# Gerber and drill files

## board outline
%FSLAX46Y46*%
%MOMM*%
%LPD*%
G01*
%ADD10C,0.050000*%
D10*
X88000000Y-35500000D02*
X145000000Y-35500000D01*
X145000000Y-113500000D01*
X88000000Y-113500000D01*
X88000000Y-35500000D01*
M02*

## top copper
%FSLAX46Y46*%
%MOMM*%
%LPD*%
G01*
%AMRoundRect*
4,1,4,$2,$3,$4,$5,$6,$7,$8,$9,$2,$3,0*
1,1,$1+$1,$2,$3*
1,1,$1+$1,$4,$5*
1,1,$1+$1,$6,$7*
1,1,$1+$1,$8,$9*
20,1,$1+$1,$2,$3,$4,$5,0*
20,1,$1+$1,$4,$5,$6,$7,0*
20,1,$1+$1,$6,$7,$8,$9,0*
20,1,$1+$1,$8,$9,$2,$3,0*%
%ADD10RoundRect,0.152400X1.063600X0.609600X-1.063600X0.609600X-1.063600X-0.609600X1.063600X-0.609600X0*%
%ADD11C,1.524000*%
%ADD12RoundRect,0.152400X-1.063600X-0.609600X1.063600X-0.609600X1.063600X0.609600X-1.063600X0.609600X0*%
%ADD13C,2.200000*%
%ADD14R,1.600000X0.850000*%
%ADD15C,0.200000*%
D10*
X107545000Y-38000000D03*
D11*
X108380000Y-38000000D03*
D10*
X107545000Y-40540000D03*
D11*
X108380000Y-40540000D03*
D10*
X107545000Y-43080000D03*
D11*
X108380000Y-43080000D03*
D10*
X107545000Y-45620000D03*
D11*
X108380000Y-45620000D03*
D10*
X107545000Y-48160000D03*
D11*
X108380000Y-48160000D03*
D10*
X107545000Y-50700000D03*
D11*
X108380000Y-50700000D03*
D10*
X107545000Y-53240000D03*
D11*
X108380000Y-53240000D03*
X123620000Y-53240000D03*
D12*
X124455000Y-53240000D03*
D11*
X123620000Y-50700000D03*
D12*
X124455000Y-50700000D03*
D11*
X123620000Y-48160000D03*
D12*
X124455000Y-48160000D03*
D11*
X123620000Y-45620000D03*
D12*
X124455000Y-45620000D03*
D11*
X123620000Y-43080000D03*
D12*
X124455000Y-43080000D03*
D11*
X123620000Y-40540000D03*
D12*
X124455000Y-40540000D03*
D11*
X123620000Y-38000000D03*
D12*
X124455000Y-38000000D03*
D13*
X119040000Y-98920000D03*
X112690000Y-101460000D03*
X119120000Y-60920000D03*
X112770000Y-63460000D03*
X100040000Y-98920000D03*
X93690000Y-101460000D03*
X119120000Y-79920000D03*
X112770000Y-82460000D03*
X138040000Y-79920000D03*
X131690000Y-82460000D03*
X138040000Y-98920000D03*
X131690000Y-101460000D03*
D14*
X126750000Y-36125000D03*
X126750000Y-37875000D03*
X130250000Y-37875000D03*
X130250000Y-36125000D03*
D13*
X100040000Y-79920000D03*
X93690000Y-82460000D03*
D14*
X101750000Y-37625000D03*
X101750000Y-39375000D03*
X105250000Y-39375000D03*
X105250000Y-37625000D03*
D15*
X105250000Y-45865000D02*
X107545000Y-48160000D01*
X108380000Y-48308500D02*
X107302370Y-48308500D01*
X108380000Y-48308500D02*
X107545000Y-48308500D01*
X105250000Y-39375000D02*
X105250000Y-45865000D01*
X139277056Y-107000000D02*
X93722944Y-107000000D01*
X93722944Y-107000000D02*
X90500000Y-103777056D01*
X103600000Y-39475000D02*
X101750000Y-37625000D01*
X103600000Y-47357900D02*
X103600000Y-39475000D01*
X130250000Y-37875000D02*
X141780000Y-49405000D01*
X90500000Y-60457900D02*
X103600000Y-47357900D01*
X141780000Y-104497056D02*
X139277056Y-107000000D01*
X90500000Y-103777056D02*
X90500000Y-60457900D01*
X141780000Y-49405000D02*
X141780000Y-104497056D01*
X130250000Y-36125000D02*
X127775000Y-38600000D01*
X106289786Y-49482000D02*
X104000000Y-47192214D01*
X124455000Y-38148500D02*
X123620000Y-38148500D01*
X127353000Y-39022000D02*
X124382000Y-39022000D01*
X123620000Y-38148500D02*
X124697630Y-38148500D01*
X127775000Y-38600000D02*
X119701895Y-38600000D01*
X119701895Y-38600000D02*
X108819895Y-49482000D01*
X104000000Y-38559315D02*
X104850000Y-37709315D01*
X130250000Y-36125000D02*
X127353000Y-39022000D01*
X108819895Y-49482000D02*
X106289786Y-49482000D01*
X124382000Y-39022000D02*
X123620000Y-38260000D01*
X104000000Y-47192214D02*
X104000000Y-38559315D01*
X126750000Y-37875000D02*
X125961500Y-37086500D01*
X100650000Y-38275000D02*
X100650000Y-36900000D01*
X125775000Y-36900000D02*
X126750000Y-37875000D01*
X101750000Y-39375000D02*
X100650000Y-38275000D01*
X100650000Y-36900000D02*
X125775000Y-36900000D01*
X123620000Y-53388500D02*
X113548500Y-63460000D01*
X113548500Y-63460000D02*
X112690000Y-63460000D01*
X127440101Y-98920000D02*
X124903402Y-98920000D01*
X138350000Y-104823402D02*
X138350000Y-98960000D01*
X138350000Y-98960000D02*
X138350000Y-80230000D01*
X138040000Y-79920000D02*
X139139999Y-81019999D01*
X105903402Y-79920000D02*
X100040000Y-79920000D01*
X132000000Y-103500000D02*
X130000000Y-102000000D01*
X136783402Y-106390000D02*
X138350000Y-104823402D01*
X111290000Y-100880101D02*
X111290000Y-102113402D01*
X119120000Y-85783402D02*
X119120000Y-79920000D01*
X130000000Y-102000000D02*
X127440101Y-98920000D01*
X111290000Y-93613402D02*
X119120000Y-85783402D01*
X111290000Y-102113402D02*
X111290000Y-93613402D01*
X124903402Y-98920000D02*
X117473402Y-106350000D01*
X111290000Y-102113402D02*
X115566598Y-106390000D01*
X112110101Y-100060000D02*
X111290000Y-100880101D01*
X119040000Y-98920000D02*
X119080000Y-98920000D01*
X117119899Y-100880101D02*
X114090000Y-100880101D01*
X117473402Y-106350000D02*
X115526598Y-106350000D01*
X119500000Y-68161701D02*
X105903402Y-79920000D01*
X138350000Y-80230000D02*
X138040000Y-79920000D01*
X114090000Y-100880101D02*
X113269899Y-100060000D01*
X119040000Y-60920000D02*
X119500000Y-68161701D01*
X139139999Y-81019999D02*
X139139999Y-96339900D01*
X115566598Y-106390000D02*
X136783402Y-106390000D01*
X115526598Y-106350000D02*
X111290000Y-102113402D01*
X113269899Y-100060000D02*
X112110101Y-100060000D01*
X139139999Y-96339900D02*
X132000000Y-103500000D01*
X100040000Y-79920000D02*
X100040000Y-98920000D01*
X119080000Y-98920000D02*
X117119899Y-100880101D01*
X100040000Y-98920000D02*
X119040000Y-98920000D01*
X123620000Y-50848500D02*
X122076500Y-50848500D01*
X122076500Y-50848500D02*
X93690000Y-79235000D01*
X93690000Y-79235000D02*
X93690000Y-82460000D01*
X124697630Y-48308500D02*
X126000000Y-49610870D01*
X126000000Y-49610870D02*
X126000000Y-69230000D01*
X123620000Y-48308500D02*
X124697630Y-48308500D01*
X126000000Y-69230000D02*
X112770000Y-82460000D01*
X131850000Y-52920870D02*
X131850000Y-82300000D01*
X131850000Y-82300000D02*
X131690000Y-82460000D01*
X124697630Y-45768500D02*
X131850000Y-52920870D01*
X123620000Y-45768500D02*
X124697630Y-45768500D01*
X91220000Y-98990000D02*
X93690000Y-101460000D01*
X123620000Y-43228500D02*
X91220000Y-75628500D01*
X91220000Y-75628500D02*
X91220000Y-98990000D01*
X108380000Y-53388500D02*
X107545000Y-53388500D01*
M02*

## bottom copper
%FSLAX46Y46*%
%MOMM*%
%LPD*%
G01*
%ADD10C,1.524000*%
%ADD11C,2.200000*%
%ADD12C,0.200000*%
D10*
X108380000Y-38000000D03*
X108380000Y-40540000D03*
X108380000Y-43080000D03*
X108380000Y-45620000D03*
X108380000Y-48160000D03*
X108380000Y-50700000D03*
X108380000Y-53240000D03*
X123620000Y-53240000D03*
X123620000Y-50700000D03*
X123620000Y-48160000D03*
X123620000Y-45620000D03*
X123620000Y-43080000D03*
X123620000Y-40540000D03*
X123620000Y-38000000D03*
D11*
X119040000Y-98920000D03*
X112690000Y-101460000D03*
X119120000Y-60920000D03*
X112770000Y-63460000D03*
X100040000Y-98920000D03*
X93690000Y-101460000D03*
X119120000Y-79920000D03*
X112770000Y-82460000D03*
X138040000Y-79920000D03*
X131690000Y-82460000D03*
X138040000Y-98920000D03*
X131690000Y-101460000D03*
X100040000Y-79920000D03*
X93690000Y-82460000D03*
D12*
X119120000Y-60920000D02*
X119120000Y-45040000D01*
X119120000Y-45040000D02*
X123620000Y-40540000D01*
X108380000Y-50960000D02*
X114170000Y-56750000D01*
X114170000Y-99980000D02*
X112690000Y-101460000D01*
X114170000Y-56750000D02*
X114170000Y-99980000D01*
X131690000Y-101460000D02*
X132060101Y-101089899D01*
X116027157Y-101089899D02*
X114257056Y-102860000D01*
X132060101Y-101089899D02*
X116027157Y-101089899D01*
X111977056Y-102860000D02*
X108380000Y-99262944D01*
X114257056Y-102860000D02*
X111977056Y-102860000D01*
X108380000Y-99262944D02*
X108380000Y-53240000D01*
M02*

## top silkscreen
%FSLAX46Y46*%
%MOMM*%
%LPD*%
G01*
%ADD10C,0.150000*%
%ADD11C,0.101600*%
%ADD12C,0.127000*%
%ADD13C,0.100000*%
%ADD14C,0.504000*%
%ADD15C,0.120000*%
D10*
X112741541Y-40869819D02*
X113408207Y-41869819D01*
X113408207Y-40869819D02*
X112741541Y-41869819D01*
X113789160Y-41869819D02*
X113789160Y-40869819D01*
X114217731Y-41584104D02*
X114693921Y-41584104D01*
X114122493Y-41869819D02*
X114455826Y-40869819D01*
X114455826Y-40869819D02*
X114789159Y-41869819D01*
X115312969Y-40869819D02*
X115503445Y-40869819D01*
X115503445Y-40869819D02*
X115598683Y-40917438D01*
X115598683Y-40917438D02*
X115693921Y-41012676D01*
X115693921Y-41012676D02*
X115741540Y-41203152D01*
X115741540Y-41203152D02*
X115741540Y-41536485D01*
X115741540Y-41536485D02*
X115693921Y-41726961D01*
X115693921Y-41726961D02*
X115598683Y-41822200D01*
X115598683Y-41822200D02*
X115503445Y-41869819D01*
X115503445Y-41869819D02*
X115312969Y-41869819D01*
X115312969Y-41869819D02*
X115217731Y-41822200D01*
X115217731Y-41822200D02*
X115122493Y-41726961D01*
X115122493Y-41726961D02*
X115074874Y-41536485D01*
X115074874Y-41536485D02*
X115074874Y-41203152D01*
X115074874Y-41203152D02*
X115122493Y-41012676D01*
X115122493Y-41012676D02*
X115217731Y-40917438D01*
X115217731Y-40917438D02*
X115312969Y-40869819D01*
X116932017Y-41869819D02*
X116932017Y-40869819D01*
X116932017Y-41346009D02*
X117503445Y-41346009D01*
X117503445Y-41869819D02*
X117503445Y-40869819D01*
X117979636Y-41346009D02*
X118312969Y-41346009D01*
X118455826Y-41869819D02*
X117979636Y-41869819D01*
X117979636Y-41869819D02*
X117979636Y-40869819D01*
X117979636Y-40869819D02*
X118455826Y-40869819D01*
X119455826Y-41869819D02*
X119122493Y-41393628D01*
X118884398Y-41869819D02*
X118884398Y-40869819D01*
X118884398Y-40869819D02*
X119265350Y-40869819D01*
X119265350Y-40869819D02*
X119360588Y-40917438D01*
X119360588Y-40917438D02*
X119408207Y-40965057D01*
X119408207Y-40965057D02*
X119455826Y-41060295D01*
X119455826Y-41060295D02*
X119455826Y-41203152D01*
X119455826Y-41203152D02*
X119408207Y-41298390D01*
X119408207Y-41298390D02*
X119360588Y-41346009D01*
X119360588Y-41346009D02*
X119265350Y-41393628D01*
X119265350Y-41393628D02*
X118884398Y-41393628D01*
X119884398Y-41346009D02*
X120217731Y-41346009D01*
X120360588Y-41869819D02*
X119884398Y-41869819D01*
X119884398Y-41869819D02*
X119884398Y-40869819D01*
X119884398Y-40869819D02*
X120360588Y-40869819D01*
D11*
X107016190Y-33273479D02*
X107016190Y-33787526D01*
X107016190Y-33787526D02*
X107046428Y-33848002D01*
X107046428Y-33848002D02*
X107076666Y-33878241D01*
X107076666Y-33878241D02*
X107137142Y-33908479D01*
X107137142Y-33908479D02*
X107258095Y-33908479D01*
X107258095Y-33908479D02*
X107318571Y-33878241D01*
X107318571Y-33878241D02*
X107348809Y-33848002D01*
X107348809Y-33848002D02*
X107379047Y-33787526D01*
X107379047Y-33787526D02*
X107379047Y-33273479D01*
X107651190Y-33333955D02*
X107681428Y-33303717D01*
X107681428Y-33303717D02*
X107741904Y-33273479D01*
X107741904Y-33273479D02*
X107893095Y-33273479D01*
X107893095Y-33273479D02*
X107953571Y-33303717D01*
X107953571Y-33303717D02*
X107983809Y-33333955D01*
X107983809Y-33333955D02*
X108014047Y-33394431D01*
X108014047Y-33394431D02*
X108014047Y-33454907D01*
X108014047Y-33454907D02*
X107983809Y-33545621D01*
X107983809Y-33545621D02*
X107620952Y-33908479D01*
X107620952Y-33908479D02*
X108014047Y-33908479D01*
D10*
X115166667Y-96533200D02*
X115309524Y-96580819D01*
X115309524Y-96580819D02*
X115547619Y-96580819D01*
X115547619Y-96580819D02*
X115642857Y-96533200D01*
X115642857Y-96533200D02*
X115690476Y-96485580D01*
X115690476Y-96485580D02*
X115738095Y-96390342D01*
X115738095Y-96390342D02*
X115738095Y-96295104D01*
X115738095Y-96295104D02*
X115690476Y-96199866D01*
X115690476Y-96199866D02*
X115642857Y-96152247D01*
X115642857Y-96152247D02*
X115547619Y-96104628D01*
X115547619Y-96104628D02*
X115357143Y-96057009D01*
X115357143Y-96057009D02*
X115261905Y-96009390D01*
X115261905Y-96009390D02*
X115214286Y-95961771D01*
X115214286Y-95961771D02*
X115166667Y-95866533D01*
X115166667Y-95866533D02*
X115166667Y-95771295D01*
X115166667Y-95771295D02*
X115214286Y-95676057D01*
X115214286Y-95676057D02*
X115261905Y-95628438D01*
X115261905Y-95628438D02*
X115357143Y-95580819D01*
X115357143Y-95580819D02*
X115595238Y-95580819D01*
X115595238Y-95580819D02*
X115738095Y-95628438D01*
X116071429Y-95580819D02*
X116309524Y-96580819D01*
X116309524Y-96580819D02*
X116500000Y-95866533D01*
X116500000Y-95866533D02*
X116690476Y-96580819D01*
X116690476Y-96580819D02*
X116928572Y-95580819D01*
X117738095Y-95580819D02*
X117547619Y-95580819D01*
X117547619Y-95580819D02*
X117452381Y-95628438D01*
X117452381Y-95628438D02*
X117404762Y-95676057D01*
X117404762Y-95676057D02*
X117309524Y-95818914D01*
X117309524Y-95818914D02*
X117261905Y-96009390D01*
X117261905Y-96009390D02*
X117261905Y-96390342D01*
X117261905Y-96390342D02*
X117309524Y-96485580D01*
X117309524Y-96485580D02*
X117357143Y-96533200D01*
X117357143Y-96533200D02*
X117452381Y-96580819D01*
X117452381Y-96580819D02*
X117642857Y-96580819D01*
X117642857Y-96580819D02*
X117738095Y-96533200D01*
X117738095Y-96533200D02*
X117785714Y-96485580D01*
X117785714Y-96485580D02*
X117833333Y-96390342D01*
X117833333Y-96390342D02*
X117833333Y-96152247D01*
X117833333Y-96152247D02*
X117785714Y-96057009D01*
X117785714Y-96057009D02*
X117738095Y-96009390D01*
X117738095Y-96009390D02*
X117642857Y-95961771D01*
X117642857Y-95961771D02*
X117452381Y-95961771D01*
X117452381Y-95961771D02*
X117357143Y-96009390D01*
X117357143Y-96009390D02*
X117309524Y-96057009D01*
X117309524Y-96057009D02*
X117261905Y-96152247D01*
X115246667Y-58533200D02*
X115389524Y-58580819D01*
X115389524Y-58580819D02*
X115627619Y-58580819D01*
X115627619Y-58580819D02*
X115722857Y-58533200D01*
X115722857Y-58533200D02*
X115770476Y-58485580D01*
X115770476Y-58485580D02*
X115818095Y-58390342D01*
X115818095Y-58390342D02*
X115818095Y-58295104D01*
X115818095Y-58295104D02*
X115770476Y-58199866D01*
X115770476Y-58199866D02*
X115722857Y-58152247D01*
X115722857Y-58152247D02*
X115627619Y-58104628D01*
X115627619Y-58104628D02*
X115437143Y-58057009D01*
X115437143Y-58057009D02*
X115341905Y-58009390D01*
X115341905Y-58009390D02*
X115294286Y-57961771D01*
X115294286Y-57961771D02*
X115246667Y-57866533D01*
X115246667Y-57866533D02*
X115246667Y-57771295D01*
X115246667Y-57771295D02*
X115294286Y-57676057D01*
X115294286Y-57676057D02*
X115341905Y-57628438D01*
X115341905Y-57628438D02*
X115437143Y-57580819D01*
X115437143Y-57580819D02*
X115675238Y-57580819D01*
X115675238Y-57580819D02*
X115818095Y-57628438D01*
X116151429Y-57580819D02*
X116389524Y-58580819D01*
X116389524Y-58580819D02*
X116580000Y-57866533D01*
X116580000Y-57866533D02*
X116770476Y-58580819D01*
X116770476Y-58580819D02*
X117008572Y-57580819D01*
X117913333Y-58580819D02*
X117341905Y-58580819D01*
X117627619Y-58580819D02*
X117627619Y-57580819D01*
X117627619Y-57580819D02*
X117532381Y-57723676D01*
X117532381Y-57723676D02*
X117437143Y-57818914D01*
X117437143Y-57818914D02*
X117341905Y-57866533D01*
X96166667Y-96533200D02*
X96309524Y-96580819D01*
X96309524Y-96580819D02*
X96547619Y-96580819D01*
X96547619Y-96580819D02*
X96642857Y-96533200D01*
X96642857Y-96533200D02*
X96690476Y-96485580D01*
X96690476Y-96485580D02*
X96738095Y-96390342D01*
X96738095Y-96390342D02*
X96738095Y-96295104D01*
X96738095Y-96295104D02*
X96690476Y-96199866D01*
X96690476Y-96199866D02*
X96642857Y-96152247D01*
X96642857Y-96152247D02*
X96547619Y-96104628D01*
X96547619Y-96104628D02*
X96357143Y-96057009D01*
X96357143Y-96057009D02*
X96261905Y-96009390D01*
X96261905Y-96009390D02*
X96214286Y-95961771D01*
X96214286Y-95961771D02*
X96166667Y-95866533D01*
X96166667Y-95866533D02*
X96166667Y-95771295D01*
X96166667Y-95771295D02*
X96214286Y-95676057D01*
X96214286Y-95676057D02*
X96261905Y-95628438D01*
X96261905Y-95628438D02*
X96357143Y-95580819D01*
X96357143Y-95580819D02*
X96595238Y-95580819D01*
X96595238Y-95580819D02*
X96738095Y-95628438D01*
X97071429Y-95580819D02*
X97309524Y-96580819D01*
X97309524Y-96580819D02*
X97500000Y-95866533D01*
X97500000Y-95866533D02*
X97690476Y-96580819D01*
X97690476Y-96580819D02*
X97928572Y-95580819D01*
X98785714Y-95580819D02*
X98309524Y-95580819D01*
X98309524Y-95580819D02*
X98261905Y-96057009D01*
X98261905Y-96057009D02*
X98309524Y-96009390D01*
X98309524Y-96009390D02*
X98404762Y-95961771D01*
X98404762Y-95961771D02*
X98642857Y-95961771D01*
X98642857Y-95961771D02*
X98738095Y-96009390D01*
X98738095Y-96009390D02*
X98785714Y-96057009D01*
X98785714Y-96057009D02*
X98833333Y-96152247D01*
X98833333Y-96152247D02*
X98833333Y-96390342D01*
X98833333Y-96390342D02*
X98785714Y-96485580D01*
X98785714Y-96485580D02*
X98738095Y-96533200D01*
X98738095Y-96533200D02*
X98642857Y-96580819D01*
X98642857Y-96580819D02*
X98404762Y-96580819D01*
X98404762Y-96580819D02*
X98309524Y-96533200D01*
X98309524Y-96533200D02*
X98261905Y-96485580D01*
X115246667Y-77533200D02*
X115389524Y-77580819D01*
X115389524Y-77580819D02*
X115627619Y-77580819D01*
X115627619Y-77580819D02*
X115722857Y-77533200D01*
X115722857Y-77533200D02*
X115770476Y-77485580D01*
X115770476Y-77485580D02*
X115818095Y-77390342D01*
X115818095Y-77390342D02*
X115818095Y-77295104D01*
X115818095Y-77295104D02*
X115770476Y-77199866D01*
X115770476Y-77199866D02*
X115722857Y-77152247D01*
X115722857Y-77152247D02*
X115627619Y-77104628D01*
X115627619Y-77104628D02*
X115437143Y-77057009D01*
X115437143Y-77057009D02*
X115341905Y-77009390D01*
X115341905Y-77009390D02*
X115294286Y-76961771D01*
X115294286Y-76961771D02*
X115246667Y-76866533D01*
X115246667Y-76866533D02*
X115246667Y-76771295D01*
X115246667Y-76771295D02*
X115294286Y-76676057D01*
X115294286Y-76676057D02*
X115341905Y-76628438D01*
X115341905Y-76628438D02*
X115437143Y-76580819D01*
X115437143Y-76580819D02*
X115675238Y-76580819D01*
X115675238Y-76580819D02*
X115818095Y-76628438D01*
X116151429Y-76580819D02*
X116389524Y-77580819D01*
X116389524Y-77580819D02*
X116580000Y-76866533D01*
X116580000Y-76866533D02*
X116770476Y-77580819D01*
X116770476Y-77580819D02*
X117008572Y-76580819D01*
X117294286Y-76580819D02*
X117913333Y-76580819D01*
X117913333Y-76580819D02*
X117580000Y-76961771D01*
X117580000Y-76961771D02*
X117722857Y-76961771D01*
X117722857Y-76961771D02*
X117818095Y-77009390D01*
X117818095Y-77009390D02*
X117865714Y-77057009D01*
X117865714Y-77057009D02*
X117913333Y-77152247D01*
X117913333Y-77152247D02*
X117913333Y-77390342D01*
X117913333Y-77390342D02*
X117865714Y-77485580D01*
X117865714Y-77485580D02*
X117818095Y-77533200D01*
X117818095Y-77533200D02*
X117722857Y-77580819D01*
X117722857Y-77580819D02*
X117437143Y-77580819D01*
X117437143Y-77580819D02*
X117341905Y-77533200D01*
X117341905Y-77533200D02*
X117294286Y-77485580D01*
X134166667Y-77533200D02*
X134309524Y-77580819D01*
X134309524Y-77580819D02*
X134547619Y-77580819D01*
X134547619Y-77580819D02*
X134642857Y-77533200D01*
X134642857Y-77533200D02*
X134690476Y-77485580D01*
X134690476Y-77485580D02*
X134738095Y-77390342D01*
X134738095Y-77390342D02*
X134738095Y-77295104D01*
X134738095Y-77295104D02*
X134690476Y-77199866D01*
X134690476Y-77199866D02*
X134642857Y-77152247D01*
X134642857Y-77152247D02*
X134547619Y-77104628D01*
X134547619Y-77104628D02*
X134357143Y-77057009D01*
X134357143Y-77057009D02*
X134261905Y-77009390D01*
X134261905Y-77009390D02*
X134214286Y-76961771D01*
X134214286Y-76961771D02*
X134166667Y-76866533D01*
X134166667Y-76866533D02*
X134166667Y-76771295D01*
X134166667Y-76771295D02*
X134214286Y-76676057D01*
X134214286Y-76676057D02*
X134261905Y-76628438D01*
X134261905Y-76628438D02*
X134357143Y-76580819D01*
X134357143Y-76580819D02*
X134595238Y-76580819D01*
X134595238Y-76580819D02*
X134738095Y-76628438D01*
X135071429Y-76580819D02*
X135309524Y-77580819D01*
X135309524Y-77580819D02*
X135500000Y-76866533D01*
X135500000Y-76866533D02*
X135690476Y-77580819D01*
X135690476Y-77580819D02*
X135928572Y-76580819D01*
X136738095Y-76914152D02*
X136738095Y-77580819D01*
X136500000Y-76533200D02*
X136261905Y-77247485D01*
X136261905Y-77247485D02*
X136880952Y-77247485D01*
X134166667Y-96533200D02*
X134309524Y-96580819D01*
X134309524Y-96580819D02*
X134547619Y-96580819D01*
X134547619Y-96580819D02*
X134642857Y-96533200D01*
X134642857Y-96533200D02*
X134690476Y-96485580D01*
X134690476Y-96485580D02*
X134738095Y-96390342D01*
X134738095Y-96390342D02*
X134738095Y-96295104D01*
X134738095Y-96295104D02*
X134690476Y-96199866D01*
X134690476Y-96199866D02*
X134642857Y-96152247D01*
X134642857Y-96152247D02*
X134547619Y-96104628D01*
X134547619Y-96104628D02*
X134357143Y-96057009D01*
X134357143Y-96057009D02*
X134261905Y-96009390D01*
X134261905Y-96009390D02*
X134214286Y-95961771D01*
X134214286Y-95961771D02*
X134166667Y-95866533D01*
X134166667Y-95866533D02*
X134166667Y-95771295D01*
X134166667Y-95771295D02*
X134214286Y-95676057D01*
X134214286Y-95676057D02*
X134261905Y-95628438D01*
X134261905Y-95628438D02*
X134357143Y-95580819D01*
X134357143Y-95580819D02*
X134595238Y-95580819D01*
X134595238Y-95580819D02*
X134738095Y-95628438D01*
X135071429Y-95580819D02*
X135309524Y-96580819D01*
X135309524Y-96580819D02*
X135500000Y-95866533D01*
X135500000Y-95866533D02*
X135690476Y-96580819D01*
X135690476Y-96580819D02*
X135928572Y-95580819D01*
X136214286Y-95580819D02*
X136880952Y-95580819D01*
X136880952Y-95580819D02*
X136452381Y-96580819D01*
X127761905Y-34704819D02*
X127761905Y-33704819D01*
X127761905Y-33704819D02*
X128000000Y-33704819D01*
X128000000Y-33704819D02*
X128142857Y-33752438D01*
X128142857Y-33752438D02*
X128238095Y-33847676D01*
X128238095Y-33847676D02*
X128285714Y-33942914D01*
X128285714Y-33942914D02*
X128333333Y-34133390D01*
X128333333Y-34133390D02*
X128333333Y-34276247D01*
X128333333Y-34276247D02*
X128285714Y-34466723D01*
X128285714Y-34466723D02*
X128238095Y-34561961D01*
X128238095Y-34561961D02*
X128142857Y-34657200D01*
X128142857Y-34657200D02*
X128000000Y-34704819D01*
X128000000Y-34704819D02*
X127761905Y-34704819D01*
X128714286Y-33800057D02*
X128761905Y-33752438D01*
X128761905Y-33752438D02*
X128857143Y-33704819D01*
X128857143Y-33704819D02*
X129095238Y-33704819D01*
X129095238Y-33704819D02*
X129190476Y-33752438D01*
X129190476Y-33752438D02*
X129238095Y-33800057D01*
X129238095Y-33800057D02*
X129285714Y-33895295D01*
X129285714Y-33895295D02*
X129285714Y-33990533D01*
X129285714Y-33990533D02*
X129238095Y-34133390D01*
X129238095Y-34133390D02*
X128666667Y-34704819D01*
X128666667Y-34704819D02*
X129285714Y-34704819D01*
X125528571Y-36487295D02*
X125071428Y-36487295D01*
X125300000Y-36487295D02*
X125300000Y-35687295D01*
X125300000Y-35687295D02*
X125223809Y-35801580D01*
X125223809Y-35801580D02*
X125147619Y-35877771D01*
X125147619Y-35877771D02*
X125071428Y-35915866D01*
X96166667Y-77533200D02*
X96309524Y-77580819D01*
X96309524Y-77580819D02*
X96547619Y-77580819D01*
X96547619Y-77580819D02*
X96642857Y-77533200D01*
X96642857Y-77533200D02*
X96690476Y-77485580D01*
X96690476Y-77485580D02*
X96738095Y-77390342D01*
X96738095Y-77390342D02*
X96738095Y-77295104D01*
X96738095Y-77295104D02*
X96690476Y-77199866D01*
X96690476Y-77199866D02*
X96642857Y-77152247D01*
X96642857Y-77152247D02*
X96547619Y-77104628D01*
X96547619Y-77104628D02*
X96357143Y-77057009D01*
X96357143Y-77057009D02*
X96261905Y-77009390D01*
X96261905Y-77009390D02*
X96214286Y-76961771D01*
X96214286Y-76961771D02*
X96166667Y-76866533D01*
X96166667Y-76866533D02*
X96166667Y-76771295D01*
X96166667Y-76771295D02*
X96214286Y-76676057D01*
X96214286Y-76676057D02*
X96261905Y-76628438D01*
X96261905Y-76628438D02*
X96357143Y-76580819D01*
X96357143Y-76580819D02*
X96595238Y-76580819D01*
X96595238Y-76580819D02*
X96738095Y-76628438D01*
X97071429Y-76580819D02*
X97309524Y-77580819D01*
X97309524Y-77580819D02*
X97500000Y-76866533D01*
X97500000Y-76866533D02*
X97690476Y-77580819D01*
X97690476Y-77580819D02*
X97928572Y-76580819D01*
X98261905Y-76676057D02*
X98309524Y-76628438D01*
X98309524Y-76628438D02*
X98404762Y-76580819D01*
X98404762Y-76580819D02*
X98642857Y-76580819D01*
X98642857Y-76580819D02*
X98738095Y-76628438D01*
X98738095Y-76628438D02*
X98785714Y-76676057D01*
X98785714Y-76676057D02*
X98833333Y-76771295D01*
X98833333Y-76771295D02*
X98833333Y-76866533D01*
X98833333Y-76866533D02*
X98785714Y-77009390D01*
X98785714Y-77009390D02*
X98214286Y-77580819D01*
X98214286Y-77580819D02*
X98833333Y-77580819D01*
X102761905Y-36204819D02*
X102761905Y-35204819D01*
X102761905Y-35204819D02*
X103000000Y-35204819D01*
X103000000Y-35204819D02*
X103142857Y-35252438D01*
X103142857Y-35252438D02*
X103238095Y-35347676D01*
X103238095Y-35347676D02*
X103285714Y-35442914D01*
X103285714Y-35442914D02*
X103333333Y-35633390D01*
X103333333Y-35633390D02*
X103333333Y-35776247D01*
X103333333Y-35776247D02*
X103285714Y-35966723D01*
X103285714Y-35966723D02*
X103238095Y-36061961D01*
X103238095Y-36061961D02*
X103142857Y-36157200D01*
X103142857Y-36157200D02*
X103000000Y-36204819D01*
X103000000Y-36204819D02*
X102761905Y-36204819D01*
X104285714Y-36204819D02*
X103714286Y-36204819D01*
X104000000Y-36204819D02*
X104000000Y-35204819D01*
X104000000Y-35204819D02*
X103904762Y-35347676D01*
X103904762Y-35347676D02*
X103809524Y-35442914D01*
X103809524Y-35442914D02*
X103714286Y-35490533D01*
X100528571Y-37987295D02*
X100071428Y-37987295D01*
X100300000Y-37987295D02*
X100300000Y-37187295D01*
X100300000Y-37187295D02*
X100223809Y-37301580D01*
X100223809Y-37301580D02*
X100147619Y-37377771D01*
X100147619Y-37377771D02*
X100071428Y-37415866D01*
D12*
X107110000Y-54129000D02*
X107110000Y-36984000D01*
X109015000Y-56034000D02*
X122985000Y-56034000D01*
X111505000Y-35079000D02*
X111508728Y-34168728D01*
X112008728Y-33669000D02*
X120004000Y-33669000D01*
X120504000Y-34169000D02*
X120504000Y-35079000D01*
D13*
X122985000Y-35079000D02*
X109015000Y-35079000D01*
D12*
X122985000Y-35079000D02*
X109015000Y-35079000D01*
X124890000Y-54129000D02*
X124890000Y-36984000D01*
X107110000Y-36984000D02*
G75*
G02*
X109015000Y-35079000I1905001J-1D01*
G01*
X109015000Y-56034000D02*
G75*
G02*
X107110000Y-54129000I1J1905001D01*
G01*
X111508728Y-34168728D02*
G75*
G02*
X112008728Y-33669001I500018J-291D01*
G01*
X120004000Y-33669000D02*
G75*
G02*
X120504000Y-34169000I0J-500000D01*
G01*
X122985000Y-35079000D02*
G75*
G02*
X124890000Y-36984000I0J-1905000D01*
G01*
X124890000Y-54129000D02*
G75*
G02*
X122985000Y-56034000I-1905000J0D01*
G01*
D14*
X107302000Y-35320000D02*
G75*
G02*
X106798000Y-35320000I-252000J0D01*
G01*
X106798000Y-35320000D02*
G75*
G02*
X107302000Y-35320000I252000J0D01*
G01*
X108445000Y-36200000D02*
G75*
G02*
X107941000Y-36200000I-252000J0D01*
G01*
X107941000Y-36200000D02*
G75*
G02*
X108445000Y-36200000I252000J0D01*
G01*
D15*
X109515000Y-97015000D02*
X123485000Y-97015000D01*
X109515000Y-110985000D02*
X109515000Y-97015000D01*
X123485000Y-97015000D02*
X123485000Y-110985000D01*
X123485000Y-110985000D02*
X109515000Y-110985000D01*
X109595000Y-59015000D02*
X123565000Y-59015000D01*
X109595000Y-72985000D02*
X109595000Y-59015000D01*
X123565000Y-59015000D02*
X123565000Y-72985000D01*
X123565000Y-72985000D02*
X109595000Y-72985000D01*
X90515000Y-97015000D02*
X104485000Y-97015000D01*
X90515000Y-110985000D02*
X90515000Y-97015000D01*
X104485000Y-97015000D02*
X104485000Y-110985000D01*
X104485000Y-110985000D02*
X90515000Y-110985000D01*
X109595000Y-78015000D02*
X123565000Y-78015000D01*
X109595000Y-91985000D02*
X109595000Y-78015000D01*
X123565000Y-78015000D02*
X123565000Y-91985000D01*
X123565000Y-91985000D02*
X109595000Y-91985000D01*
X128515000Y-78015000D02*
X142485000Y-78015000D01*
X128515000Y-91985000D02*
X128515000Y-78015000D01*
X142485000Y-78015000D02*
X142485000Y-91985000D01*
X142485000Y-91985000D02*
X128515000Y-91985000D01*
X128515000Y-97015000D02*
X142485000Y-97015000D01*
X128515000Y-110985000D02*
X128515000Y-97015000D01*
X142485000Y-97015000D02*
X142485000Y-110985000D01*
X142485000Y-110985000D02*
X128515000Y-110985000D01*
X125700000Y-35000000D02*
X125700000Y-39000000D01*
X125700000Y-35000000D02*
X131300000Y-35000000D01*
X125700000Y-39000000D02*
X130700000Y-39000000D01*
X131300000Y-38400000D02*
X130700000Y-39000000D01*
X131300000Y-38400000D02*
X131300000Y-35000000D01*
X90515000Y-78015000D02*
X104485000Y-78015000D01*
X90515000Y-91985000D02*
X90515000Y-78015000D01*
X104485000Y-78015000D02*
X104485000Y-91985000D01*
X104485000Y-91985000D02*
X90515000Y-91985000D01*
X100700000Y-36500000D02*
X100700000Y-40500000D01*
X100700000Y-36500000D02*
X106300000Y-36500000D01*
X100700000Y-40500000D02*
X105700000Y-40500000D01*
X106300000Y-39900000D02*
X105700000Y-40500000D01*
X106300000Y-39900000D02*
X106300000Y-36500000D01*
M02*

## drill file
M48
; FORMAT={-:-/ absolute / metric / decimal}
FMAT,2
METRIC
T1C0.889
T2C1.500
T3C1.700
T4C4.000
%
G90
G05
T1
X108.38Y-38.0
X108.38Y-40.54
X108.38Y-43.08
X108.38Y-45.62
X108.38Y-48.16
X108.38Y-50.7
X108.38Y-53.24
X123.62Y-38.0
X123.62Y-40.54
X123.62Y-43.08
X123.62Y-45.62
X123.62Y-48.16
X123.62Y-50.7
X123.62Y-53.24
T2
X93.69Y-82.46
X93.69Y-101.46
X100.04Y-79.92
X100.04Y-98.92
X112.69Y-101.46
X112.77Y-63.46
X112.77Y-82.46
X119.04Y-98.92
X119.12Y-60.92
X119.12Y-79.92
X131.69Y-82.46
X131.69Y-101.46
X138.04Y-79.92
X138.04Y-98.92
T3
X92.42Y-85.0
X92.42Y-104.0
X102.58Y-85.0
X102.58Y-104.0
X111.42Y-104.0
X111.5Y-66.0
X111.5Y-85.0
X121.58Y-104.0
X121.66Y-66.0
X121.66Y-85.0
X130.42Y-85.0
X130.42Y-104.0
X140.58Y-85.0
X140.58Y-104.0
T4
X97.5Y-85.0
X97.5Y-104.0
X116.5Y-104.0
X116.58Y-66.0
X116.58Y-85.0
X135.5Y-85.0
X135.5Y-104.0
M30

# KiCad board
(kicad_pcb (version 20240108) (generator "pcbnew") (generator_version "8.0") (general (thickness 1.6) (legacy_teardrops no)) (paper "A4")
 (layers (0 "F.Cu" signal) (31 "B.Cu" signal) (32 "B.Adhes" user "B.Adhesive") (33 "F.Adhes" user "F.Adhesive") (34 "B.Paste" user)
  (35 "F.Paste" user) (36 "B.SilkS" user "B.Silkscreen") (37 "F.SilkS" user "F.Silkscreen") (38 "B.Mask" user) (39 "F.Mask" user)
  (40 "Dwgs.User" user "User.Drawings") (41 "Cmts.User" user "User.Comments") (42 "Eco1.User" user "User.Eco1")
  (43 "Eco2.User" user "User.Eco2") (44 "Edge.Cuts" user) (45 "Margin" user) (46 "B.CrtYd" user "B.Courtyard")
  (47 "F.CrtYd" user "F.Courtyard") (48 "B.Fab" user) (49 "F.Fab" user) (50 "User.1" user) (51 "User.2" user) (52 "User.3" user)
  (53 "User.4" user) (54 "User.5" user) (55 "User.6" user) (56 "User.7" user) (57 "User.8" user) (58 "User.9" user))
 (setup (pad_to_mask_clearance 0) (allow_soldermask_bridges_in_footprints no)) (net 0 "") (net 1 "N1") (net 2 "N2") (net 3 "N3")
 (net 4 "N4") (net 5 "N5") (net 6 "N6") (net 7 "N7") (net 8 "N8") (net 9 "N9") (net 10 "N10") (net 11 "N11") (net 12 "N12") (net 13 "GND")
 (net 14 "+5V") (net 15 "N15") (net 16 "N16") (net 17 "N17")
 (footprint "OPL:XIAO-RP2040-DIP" (layer "F.Cu") (at 116 45.62)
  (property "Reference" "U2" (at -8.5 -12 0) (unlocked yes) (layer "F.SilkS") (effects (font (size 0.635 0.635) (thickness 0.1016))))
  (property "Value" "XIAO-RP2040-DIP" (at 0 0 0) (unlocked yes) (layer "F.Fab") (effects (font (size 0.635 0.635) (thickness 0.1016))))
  (fp_line (start -8.89 8.509) (end -8.89 -8.636) (stroke (width 0.127) (type solid)) (layer "F.SilkS"))
  (fp_line (start -6.985 10.414) (end 6.985 10.414) (stroke (width 0.127) (type solid)) (layer "F.SilkS"))
  (fp_line (start -4.495 -10.541) (end -4.491272 -11.451272) (stroke (width 0.127) (type solid)) (layer "F.SilkS"))
  (fp_line (start -3.991272 -11.951) (end 4.004 -11.951) (stroke (width 0.127) (type solid)) (layer "F.SilkS"))
  (fp_line (start 4.504 -11.451) (end 4.504 -10.541) (stroke (width 0.127) (type solid)) (layer "F.SilkS"))
  (fp_line (start 6.985 -10.541) (end -6.985 -10.541) (stroke (width 0.1) (type solid)) (layer "F.SilkS"))
  (fp_line (start 6.985 -10.541) (end -6.985 -10.541) (stroke (width 0.127) (type solid)) (layer "F.SilkS"))
  (fp_line (start 8.89 8.509) (end 8.89 -8.636) (stroke (width 0.127) (type solid)) (layer "F.SilkS"))
  (fp_arc (start -8.89 -8.636) (mid -8.332038 -9.983038) (end -6.985 -10.541) (stroke (width 0.127) (type solid)) (layer "F.SilkS"))
  (fp_arc (start -6.985 10.414) (mid -8.332038 9.856038) (end -8.89 8.509) (stroke (width 0.127) (type solid)) (layer "F.SilkS"))
  (fp_arc (start -4.491272 -11.451272) (mid -4.344724 -11.804644) (end -3.991272 -11.951) (stroke (width 0.127) (type default))
   (layer "F.SilkS"))
  (fp_arc (start 4.004 -11.951) (mid 4.357553 -11.804553) (end 4.504 -11.451) (stroke (width 0.127) (type default)) (layer "F.SilkS"))
  (fp_arc (start 6.985 -10.541) (mid 8.332038 -9.983038) (end 8.89 -8.636) (stroke (width 0.127) (type solid)) (layer "F.SilkS"))
  (fp_arc (start 8.89 8.509) (mid 8.332038 9.856038) (end 6.985 10.414) (stroke (width 0.127) (type solid)) (layer "F.SilkS"))
  (fp_circle (center -8.95 -10.3) (end -8.95 -10.554) (stroke (width 0.5) (type solid)) (fill solid) (layer "F.SilkS"))
  (fp_circle (center -7.807 -9.42) (end -7.807 -9.674) (stroke (width 0.5) (type solid)) (fill solid) (layer "F.SilkS"))
  (pad "1" smd roundrect (at -8.455 -7.62 180) (size 2.432 1.524) (layers "F.Cu" "F.Mask") (roundrect_rratio 0.1) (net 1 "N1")
   (thermal_bridge_angle 45))
  (pad "1" thru_hole circle (at -7.62 -7.62 180) (size 1.524 1.524) (drill 0.889) (layers "*.Cu" "*.Mask") (remove_unused_layers no)
   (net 1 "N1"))
  (pad "2" smd roundrect (at -8.455 -5.08 180) (size 2.432 1.524) (layers "F.Cu" "F.Mask") (roundrect_rratio 0.1) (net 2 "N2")
   (thermal_bridge_angle 45))
  (pad "2" thru_hole circle (at -7.62 -5.08 180) (size 1.524 1.524) (drill 0.889) (layers "*.Cu" "*.Mask") (remove_unused_layers no)
   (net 2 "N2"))
  (pad "3" smd roundrect (at -8.455 -2.54 180) (size 2.432 1.524) (layers "F.Cu" "F.Mask") (roundrect_rratio 0.1) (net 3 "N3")
   (thermal_bridge_angle 45))
  (pad "3" thru_hole circle (at -7.62 -2.54 180) (size 1.524 1.524) (drill 0.889) (layers "*.Cu" "*.Mask") (remove_unused_layers no)
   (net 3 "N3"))
  (pad "4" smd roundrect (at -8.455 0 180) (size 2.432 1.524) (layers "F.Cu" "F.Mask") (roundrect_rratio 0.1) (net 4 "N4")
   (thermal_bridge_angle 45))
  (pad "4" thru_hole circle (at -7.62 0 180) (size 1.524 1.524) (drill 0.889) (layers "*.Cu" "*.Mask") (remove_unused_layers no)
   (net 4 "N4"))
  (pad "5" smd roundrect (at -8.455 2.54 180) (size 2.432 1.524) (layers "F.Cu" "F.Mask") (roundrect_rratio 0.1) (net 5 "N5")
   (thermal_bridge_angle 45))
  (pad "5" thru_hole circle (at -7.62 2.54 180) (size 1.524 1.524) (drill 0.889) (layers "*.Cu" "*.Mask") (remove_unused_layers no)
   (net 5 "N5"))
  (pad "6" smd roundrect (at -8.455 5.08 180) (size 2.432 1.524) (layers "F.Cu" "F.Mask") (roundrect_rratio 0.1) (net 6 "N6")
   (thermal_bridge_angle 45))
  (pad "6" thru_hole circle (at -7.62 5.08 180) (size 1.524 1.524) (drill 0.889) (layers "*.Cu" "*.Mask") (remove_unused_layers no)
   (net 6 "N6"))
  (pad "7" smd roundrect (at -8.455 7.62 180) (size 2.432 1.524) (layers "F.Cu" "F.Mask") (roundrect_rratio 0.1) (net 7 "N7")
   (thermal_bridge_angle 45))
  (pad "7" thru_hole circle (at -7.62 7.62 180) (size 1.524 1.524) (drill 0.889) (layers "*.Cu" "*.Mask") (remove_unused_layers no)
   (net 7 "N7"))
  (pad "8" thru_hole circle (at 7.62 7.62) (size 1.524 1.524) (drill 0.889) (layers "*.Cu" "*.Mask") (remove_unused_layers no) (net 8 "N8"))
  (pad "8" smd roundrect (at 8.455 7.62) (size 2.432 1.524) (layers "F.Cu" "F.Mask") (roundrect_rratio 0.1) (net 8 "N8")
   (thermal_bridge_angle 45))
  (pad "9" thru_hole circle (at 7.62 5.08) (size 1.524 1.524) (drill 0.889) (layers "*.Cu" "*.Mask") (remove_unused_layers no) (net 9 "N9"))
  (pad "9" smd roundrect (at 8.455 5.08) (size 2.432 1.524) (layers "F.Cu" "F.Mask") (roundrect_rratio 0.1) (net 9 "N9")
   (thermal_bridge_angle 45))
  (pad "10" thru_hole circle (at 7.62 2.54) (size 1.524 1.524) (drill 0.889) (layers "*.Cu" "*.Mask") (remove_unused_layers no)
   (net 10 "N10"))
  (pad "10" smd roundrect (at 8.455 2.54) (size 2.432 1.524) (layers "F.Cu" "F.Mask") (roundrect_rratio 0.1) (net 10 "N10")
   (thermal_bridge_angle 45))
  (pad "11" thru_hole circle (at 7.62 0) (size 1.524 1.524) (drill 0.889) (layers "*.Cu" "*.Mask") (remove_unused_layers no) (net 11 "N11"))
  (pad "11" smd roundrect (at 8.455 0) (size 2.432 1.524) (layers "F.Cu" "F.Mask") (roundrect_rratio 0.1) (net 11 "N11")
   (thermal_bridge_angle 45))
  (pad "12" thru_hole circle (at 7.62 -2.54) (size 1.524 1.524) (drill 0.889) (layers "*.Cu" "*.Mask") (remove_unused_layers no)
   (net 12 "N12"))
  (pad "12" smd roundrect (at 8.455 -2.54) (size 2.432 1.524) (layers "F.Cu" "F.Mask") (roundrect_rratio 0.1) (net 12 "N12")
   (thermal_bridge_angle 45))
  (pad "13" thru_hole circle (at 7.62 -5.08) (size 1.524 1.524) (drill 0.889) (layers "*.Cu" "*.Mask") (remove_unused_layers no)
   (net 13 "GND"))
  (pad "13" smd roundrect (at 8.455 -5.08) (size 2.432 1.524) (layers "F.Cu" "F.Mask") (roundrect_rratio 0.1) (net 13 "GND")
   (thermal_bridge_angle 45))
  (pad "14" thru_hole circle (at 7.62 -7.62) (size 1.524 1.524) (drill 0.889) (layers "*.Cu" "*.Mask") (remove_unused_layers no)
   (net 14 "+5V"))
  (pad "14" smd roundrect (at 8.455 -7.62) (size 2.432 1.524) (layers "F.Cu" "F.Mask") (roundrect_rratio 0.1) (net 14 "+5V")
   (thermal_bridge_angle 45)))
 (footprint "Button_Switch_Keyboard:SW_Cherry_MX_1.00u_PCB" (layer "F.Cu") (at 119.04 98.92)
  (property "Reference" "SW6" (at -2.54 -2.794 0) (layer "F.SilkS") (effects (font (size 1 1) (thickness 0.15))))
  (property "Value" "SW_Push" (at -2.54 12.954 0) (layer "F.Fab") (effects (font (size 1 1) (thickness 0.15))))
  (fp_line (start -9.525 -1.905) (end 4.445 -1.905) (stroke (width 0.12) (type solid)) (layer "F.SilkS"))
  (fp_line (start -9.525 12.065) (end -9.525 -1.905) (stroke (width 0.12) (type solid)) (layer "F.SilkS"))
  (fp_line (start 4.445 -1.905) (end 4.445 12.065) (stroke (width 0.12) (type solid)) (layer "F.SilkS"))
  (fp_line (start 4.445 12.065) (end -9.525 12.065) (stroke (width 0.12) (type solid)) (layer "F.SilkS"))
  (pad "" np_thru_hole circle (at -7.62 5.08) (size 1.7 1.7) (drill 1.7) (layers "*.Cu" "*.Mask"))
  (pad "" np_thru_hole circle (at -2.54 5.08) (size 4 4) (drill 4) (layers "*.Cu" "*.Mask"))
  (pad "" np_thru_hole circle (at 2.54 5.08) (size 1.7 1.7) (drill 1.7) (layers "*.Cu" "*.Mask"))
  (pad "1" thru_hole circle (at 0 0) (size 2.2 2.2) (drill 1.5) (layers "*.Cu" "*.Mask") (remove_unused_layers no) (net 13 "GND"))
  (pad "2" thru_hole circle (at -6.35 2.54) (size 2.2 2.2) (drill 1.5) (layers "*.Cu" "*.Mask") (remove_unused_layers no) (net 6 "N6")))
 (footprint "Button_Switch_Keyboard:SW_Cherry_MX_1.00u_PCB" (layer "F.Cu") (at 119.12 60.92)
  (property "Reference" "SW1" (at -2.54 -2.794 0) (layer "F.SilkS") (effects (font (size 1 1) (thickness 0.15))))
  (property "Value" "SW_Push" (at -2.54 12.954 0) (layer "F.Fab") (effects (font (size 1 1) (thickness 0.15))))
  (fp_line (start -9.525 -1.905) (end 4.445 -1.905) (stroke (width 0.12) (type solid)) (layer "F.SilkS"))
  (fp_line (start -9.525 12.065) (end -9.525 -1.905) (stroke (width 0.12) (type solid)) (layer "F.SilkS"))
  (fp_line (start 4.445 -1.905) (end 4.445 12.065) (stroke (width 0.12) (type solid)) (layer "F.SilkS"))
  (fp_line (start 4.445 12.065) (end -9.525 12.065) (stroke (width 0.12) (type solid)) (layer "F.SilkS"))
  (pad "" np_thru_hole circle (at -7.62 5.08) (size 1.7 1.7) (drill 1.7) (layers "*.Cu" "*.Mask"))
  (pad "" np_thru_hole circle (at -2.54 5.08) (size 4 4) (drill 4) (layers "*.Cu" "*.Mask"))
  (pad "" np_thru_hole circle (at 2.54 5.08) (size 1.7 1.7) (drill 1.7) (layers "*.Cu" "*.Mask"))
  (pad "1" thru_hole circle (at 0 0) (size 2.2 2.2) (drill 1.5) (layers "*.Cu" "*.Mask") (remove_unused_layers no) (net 13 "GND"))
  (pad "2" thru_hole circle (at -6.35 2.54) (size 2.2 2.2) (drill 1.5) (layers "*.Cu" "*.Mask") (remove_unused_layers no) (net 8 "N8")))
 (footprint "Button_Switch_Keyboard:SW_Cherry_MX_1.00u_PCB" (layer "F.Cu") (at 100.04 98.92)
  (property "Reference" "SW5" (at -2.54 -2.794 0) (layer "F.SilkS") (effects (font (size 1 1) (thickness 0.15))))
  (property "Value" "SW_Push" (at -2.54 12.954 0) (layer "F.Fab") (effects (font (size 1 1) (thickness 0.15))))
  (fp_line (start -9.525 -1.905) (end 4.445 -1.905) (stroke (width 0.12) (type solid)) (layer "F.SilkS"))
  (fp_line (start -9.525 12.065) (end -9.525 -1.905) (stroke (width 0.12) (type solid)) (layer "F.SilkS"))
  (fp_line (start 4.445 -1.905) (end 4.445 12.065) (stroke (width 0.12) (type solid)) (layer "F.SilkS"))
  (fp_line (start 4.445 12.065) (end -9.525 12.065) (stroke (width 0.12) (type solid)) (layer "F.SilkS"))
  (pad "" np_thru_hole circle (at -7.62 5.08) (size 1.7 1.7) (drill 1.7) (layers "*.Cu" "*.Mask"))
  (pad "" np_thru_hole circle (at -2.54 5.08) (size 4 4) (drill 4) (layers "*.Cu" "*.Mask"))
  (pad "" np_thru_hole circle (at 2.54 5.08) (size 1.7 1.7) (drill 1.7) (layers "*.Cu" "*.Mask"))
  (pad "1" thru_hole circle (at 0 0) (size 2.2 2.2) (drill 1.5) (layers "*.Cu" "*.Mask") (remove_unused_layers no) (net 13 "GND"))
  (pad "2" thru_hole circle (at -6.35 2.54) (size 2.2 2.2) (drill 1.5) (layers "*.Cu" "*.Mask") (remove_unused_layers no) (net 12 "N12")))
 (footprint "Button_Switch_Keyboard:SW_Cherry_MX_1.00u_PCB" (layer "F.Cu") (at 119.12 79.92)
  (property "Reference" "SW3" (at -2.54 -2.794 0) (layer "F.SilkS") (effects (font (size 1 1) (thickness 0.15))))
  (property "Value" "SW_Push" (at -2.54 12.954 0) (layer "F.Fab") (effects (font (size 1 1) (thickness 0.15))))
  (fp_line (start -9.525 -1.905) (end 4.445 -1.905) (stroke (width 0.12) (type solid)) (layer "F.SilkS"))
  (fp_line (start -9.525 12.065) (end -9.525 -1.905) (stroke (width 0.12) (type solid)) (layer "F.SilkS"))
  (fp_line (start 4.445 -1.905) (end 4.445 12.065) (stroke (width 0.12) (type solid)) (layer "F.SilkS"))
  (fp_line (start 4.445 12.065) (end -9.525 12.065) (stroke (width 0.12) (type solid)) (layer "F.SilkS"))
  (pad "" np_thru_hole circle (at -7.62 5.08) (size 1.7 1.7) (drill 1.7) (layers "*.Cu" "*.Mask"))
  (pad "" np_thru_hole circle (at -2.54 5.08) (size 4 4) (drill 4) (layers "*.Cu" "*.Mask"))
  (pad "" np_thru_hole circle (at 2.54 5.08) (size 1.7 1.7) (drill 1.7) (layers "*.Cu" "*.Mask"))
  (pad "1" thru_hole circle (at 0 0) (size 2.2 2.2) (drill 1.5) (layers "*.Cu" "*.Mask") (remove_unused_layers no) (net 13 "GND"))
  (pad "2" thru_hole circle (at -6.35 2.54) (size 2.2 2.2) (drill 1.5) (layers "*.Cu" "*.Mask") (remove_unused_layers no) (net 10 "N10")))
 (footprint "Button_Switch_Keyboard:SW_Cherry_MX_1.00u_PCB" (layer "F.Cu") (at 138.04 79.92)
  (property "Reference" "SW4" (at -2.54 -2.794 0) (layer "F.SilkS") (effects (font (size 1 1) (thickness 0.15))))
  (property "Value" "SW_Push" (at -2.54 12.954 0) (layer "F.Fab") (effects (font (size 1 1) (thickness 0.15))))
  (fp_line (start -9.525 -1.905) (end 4.445 -1.905) (stroke (width 0.12) (type solid)) (layer "F.SilkS"))
  (fp_line (start -9.525 12.065) (end -9.525 -1.905) (stroke (width 0.12) (type solid)) (layer "F.SilkS"))
  (fp_line (start 4.445 -1.905) (end 4.445 12.065) (stroke (width 0.12) (type solid)) (layer "F.SilkS"))
  (fp_line (start 4.445 12.065) (end -9.525 12.065) (stroke (width 0.12) (type solid)) (layer "F.SilkS"))
  (pad "" np_thru_hole circle (at -7.62 5.08) (size 1.7 1.7) (drill 1.7) (layers "*.Cu" "*.Mask"))
  (pad "" np_thru_hole circle (at -2.54 5.08) (size 4 4) (drill 4) (layers "*.Cu" "*.Mask"))
  (pad "" np_thru_hole circle (at 2.54 5.08) (size 1.7 1.7) (drill 1.7) (layers "*.Cu" "*.Mask"))
  (pad "1" thru_hole circle (at 0 0) (size 2.2 2.2) (drill 1.5) (layers "*.Cu" "*.Mask") (remove_unused_layers no) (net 13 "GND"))
  (pad "2" thru_hole circle (at -6.35 2.54) (size 2.2 2.2) (drill 1.5) (layers "*.Cu" "*.Mask") (remove_unused_layers no) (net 11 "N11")))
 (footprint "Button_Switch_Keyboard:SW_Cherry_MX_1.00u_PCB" (layer "F.Cu") (at 138.04 98.92)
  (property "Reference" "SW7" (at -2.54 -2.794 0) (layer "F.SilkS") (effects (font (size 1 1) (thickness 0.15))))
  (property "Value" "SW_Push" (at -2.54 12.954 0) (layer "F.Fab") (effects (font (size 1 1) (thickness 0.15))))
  (fp_line (start -9.525 -1.905) (end 4.445 -1.905) (stroke (width 0.12) (type solid)) (layer "F.SilkS"))
  (fp_line (start -9.525 12.065) (end -9.525 -1.905) (stroke (width 0.12) (type solid)) (layer "F.SilkS"))
  (fp_line (start 4.445 -1.905) (end 4.445 12.065) (stroke (width 0.12) (type solid)) (layer "F.SilkS"))
  (fp_line (start 4.445 12.065) (end -9.525 12.065) (stroke (width 0.12) (type solid)) (layer "F.SilkS"))
  (pad "" np_thru_hole circle (at -7.62 5.08) (size 1.7 1.7) (drill 1.7) (layers "*.Cu" "*.Mask"))
  (pad "" np_thru_hole circle (at -2.54 5.08) (size 4 4) (drill 4) (layers "*.Cu" "*.Mask"))
  (pad "" np_thru_hole circle (at 2.54 5.08) (size 1.7 1.7) (drill 1.7) (layers "*.Cu" "*.Mask"))
  (pad "1" thru_hole circle (at 0 0) (size 2.2 2.2) (drill 1.5) (layers "*.Cu" "*.Mask") (remove_unused_layers no) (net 13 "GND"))
  (pad "2" thru_hole circle (at -6.35 2.54) (size 2.2 2.2) (drill 1.5) (layers "*.Cu" "*.Mask") (remove_unused_layers no) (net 7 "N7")))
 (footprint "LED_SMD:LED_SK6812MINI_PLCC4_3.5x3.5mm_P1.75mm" (layer "F.Cu") (at 128.5 37)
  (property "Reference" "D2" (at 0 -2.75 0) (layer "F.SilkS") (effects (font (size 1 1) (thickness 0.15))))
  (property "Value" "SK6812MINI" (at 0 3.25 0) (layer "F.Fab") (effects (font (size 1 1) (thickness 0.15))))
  (fp_line (start -2.8 -2) (end -2.8 2) (stroke (width 0.12) (type default)) (layer "F.SilkS"))
  (fp_line (start -2.8 -2) (end 2.8 -2) (stroke (width 0.12) (type solid)) (layer "F.SilkS"))
  (fp_line (start -2.8 2) (end 2.2 2) (stroke (width 0.12) (type solid)) (layer "F.SilkS"))
  (fp_line (start 2.8 1.4) (end 2.2 2) (stroke (width 0.12) (type default)) (layer "F.SilkS"))
  (fp_line (start 2.8 1.4) (end 2.8 -2) (stroke (width 0.12) (type solid)) (layer "F.SilkS"))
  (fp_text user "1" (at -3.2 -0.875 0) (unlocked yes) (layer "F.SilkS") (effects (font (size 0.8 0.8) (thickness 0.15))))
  (pad "1" smd rect (at -1.75 -0.875) (size 1.6 0.85) (layers "F.Cu" "F.Paste" "F.Mask") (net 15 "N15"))
  (pad "2" smd rect (at -1.75 0.875) (size 1.6 0.85) (layers "F.Cu" "F.Paste" "F.Mask") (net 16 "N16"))
  (pad "3" smd rect (at 1.75 0.875) (size 1.6 0.85) (layers "F.Cu" "F.Paste" "F.Mask") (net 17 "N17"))
  (pad "4" smd rect (at 1.75 -0.875) (size 1.6 0.85) (layers "F.Cu" "F.Paste" "F.Mask") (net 14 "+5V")))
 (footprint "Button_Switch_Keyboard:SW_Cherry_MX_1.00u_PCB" (layer "F.Cu") (at 100.04 79.92)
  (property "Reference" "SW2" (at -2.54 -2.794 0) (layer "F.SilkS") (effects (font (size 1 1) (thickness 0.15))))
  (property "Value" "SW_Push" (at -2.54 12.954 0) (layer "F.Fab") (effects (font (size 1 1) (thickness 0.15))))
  (fp_line (start -9.525 -1.905) (end 4.445 -1.905) (stroke (width 0.12) (type solid)) (layer "F.SilkS"))
  (fp_line (start -9.525 12.065) (end -9.525 -1.905) (stroke (width 0.12) (type solid)) (layer "F.SilkS"))
  (fp_line (start 4.445 -1.905) (end 4.445 12.065) (stroke (width 0.12) (type solid)) (layer "F.SilkS"))
  (fp_line (start 4.445 12.065) (end -9.525 12.065) (stroke (width 0.12) (type solid)) (layer "F.SilkS"))
  (pad "" np_thru_hole circle (at -7.62 5.08) (size 1.7 1.7) (drill 1.7) (layers "*.Cu" "*.Mask"))
  (pad "" np_thru_hole circle (at -2.54 5.08) (size 4 4) (drill 4) (layers "*.Cu" "*.Mask"))
  (pad "" np_thru_hole circle (at 2.54 5.08) (size 1.7 1.7) (drill 1.7) (layers "*.Cu" "*.Mask"))
  (pad "1" thru_hole circle (at 0 0) (size 2.2 2.2) (drill 1.5) (layers "*.Cu" "*.Mask") (remove_unused_layers no) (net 13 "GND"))
  (pad "2" thru_hole circle (at -6.35 2.54) (size 2.2 2.2) (drill 1.5) (layers "*.Cu" "*.Mask") (remove_unused_layers no) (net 9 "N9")))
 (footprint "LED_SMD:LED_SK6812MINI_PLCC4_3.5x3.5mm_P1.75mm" (layer "F.Cu") (at 103.5 38.5)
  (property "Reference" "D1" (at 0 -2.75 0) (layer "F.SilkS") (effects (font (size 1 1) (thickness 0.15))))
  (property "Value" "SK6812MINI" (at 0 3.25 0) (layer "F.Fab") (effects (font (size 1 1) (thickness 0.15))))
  (fp_line (start -2.8 -2) (end -2.8 2) (stroke (width 0.12) (type default)) (layer "F.SilkS"))
  (fp_line (start -2.8 -2) (end 2.8 -2) (stroke (width 0.12) (type solid)) (layer "F.SilkS"))
  (fp_line (start -2.8 2) (end 2.2 2) (stroke (width 0.12) (type solid)) (layer "F.SilkS"))
  (fp_line (start 2.8 1.4) (end 2.2 2) (stroke (width 0.12) (type default)) (layer "F.SilkS"))
  (fp_line (start 2.8 1.4) (end 2.8 -2) (stroke (width 0.12) (type solid)) (layer "F.SilkS"))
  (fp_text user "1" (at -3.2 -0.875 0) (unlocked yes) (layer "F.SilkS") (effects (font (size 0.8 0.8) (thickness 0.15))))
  (pad "1" smd rect (at -1.75 -0.875) (size 1.6 0.85) (layers "F.Cu" "F.Paste" "F.Mask") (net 17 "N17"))
  (pad "2" smd rect (at -1.75 0.875) (size 1.6 0.85) (layers "F.Cu" "F.Paste" "F.Mask") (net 16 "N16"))
  (pad "3" smd rect (at 1.75 0.875) (size 1.6 0.85) (layers "F.Cu" "F.Paste" "F.Mask") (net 5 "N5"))
  (pad "4" smd rect (at 1.75 -0.875) (size 1.6 0.85) (layers "F.Cu" "F.Paste" "F.Mask") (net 14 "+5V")))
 (gr_rect (start 88 35.5) (end 145 113.5) (stroke (width 0.05) (type default)) (fill none) (layer "Edge.Cuts"))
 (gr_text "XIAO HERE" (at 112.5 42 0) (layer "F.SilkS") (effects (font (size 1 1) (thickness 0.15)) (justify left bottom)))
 (segment (start 105.25 45.865) (end 107.545 48.16) (width 0.2) (layer "F.Cu") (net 5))
 (segment (start 108.38 48.3085) (end 107.30237 48.3085) (width 0.2) (layer "F.Cu") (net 5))
 (segment (start 108.38 48.3085) (end 107.545 48.3085) (width 0.2) (layer "F.Cu") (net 5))
 (segment (start 105.25 39.375) (end 105.25 45.865) (width 0.2) (layer "F.Cu") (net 5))
 (segment (start 139.277056 107) (end 93.722944 107) (width 0.2) (layer "F.Cu") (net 17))
 (segment (start 93.722944 107) (end 90.5 103.777056) (width 0.2) (layer "F.Cu") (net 17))
 (segment (start 103.6 39.475) (end 101.75 37.625) (width 0.2) (layer "F.Cu") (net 17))
 (segment (start 103.6 47.3579) (end 103.6 39.475) (width 0.2) (layer "F.Cu") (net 17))
 (segment (start 130.25 37.875) (end 141.78 49.405) (width 0.2) (layer "F.Cu") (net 17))
 (segment (start 90.5 60.4579) (end 103.6 47.3579) (width 0.2) (layer "F.Cu") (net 17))
 (segment (start 141.78 104.497056) (end 139.277056 107) (width 0.2) (layer "F.Cu") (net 17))
 (segment (start 90.5 103.777056) (end 90.5 60.4579) (width 0.2) (layer "F.Cu") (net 17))
 (segment (start 141.78 49.405) (end 141.78 104.497056) (width 0.2) (layer "F.Cu") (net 17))
 (segment (start 130.25 36.125) (end 127.775 38.6) (width 0.2) (layer "F.Cu") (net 14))
 (segment (start 106.289786 49.482) (end 104 47.192214) (width 0.2) (layer "F.Cu") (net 14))
 (segment (start 124.455 38.1485) (end 123.62 38.1485) (width 0.2) (layer "F.Cu") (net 14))
 (segment (start 127.353 39.022) (end 124.382 39.022) (width 0.2) (layer "F.Cu") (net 14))
 (segment (start 123.62 38.1485) (end 124.69763 38.1485) (width 0.2) (layer "F.Cu") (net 14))
 (segment (start 127.775 38.6) (end 119.701895 38.6) (width 0.2) (layer "F.Cu") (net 14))
 (segment (start 119.701895 38.6) (end 108.819895 49.482) (width 0.2) (layer "F.Cu") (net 14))
 (segment (start 104 38.559315) (end 104.85 37.709315) (width 0.2) (layer "F.Cu") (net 14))
 (segment (start 130.25 36.125) (end 127.353 39.022) (width 0.2) (layer "F.Cu") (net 14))
 (segment (start 108.819895 49.482) (end 106.289786 49.482) (width 0.2) (layer "F.Cu") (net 14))
 (segment (start 124.382 39.022) (end 123.62 38.26) (width 0.2) (layer "F.Cu") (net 14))
 (segment (start 104 47.192214) (end 104 38.559315) (width 0.2) (layer "F.Cu") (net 14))
 (segment (start 126.75 37.875) (end 125.9615 37.0865) (width 0.2) (layer "F.Cu") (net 16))
 (segment (start 100.65 38.275) (end 100.65 36.9) (width 0.2) (layer "F.Cu") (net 16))
 (segment (start 125.775 36.9) (end 126.75 37.875) (width 0.2) (layer "F.Cu") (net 16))
 (segment (start 101.75 39.375) (end 100.65 38.275) (width 0.2) (layer "F.Cu") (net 16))
 (segment (start 100.65 36.9) (end 125.775 36.9) (width 0.2) (layer "F.Cu") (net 16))
 (segment (start 123.62 53.3885) (end 113.5485 63.46) (width 0.2) (layer "F.Cu") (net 8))
 (segment (start 113.5485 63.46) (end 112.69 63.46) (width 0.2) (layer "F.Cu") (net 8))
 (segment (start 127.440101 98.92) (end 124.903402 98.92) (width 0.2) (layer "F.Cu") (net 13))
 (segment (start 138.35 104.823402) (end 138.35 98.96) (width 0.2) (layer "F.Cu") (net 13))
 (segment (start 138.35 98.96) (end 138.35 80.23) (width 0.2) (layer "F.Cu") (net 13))
 (segment (start 138.04 79.92) (end 139.139999 81.019999) (width 0.2) (layer "F.Cu") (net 13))
 (segment (start 105.903402 79.92) (end 100.04 79.92) (width 0.2) (layer "F.Cu") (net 13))
 (segment (start 132 103.5) (end 130 102) (width 0.2) (layer "F.Cu") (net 13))
 (segment (start 136.783402 106.39) (end 138.35 104.823402) (width 0.2) (layer "F.Cu") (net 13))
 (segment (start 111.29 100.880101) (end 111.29 102.113402) (width 0.2) (layer "F.Cu") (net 13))
 (segment (start 119.12 85.783402) (end 119.12 79.92) (width 0.2) (layer "F.Cu") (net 13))
 (segment (start 130 102) (end 127.440101 98.92) (width 0.2) (layer "F.Cu") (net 13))
 (segment (start 111.29 93.613402) (end 119.12 85.783402) (width 0.2) (layer "F.Cu") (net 13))
 (segment (start 111.29 102.113402) (end 111.29 93.613402) (width 0.2) (layer "F.Cu") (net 13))
 (segment (start 124.903402 98.92) (end 117.473402 106.35) (width 0.2) (layer "F.Cu") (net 13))
 (segment (start 111.29 102.113402) (end 115.566598 106.39) (width 0.2) (layer "F.Cu") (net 13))
 (segment (start 112.110101 100.06) (end 111.29 100.880101) (width 0.2) (layer "F.Cu") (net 13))
 (segment (start 119.04 98.92) (end 119.08 98.92) (width 0.2) (layer "F.Cu") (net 13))
 (segment (start 117.119899 100.880101) (end 114.09 100.880101) (width 0.2) (layer "F.Cu") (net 13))
 (segment (start 117.473402 106.35) (end 115.526598 106.35) (width 0.2) (layer "F.Cu") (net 13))
 (segment (start 119.5 68.161701) (end 105.903402 79.92) (width 0.2) (layer "F.Cu") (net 13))
 (segment (start 138.35 80.23) (end 138.04 79.92) (width 0.2) (layer "F.Cu") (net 13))
 (segment (start 114.09 100.880101) (end 113.269899 100.06) (width 0.2) (layer "F.Cu") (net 13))
 (segment (start 119.04 60.92) (end 119.5 68.161701) (width 0.2) (layer "F.Cu") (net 13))
 (segment (start 139.139999 81.019999) (end 139.139999 96.3399) (width 0.2) (layer "F.Cu") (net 13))
 (segment (start 115.566598 106.39) (end 136.783402 106.39) (width 0.2) (layer "F.Cu") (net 13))
 (segment (start 115.526598 106.35) (end 111.29 102.113402) (width 0.2) (layer "F.Cu") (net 13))
 (segment (start 113.269899 100.06) (end 112.110101 100.06) (width 0.2) (layer "F.Cu") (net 13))
 (segment (start 139.139999 96.3399) (end 132 103.5) (width 0.2) (layer "F.Cu") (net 13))
 (segment (start 100.04 79.92) (end 100.04 98.92) (width 0.2) (layer "F.Cu") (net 13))
 (segment (start 119.08 98.92) (end 117.119899 100.880101) (width 0.2) (layer "F.Cu") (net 13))
 (segment (start 100.04 98.92) (end 119.04 98.92) (width 0.2) (layer "F.Cu") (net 13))
 (segment (start 119.12 60.92) (end 119.12 45.04) (width 0.2) (layer "B.Cu") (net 13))
 (segment (start 119.12 45.04) (end 123.62 40.54) (width 0.2) (layer "B.Cu") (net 13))
 (segment (start 123.62 50.8485) (end 122.0765 50.8485) (width 0.2) (layer "F.Cu") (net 9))
 (segment (start 122.0765 50.8485) (end 93.69 79.235) (width 0.2) (layer "F.Cu") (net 9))
 (segment (start 93.69 79.235) (end 93.69 82.46) (width 0.2) (layer "F.Cu") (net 9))
 (segment (start 124.69763 48.3085) (end 126 49.61087) (width 0.2) (layer "F.Cu") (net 10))
 (segment (start 126 49.61087) (end 126 69.23) (width 0.2) (layer "F.Cu") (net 10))
 (segment (start 123.62 48.3085) (end 124.69763 48.3085) (width 0.2) (layer "F.Cu") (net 10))
 (segment (start 126 69.23) (end 112.77 82.46) (width 0.2) (layer "F.Cu") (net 10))
 (segment (start 131.85 52.92087) (end 131.85 82.3) (width 0.2) (layer "F.Cu") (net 11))
 (segment (start 131.85 82.3) (end 131.69 82.46) (width 0.2) (layer "F.Cu") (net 11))
 (segment (start 124.69763 45.7685) (end 131.85 52.92087) (width 0.2) (layer "F.Cu") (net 11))
 (segment (start 123.62 45.7685) (end 124.69763 45.7685) (width 0.2) (layer "F.Cu") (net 11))
 (segment (start 91.22 98.99) (end 93.69 101.46) (width 0.2) (layer "F.Cu") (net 12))
 (segment (start 123.62 43.2285) (end 91.22 75.6285) (width 0.2) (layer "F.Cu") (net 12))
 (segment (start 91.22 75.6285) (end 91.22 98.99) (width 0.2) (layer "F.Cu") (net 12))
 (segment (start 108.38 50.96) (end 114.17 56.75) (width 0.2) (layer "B.Cu") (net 6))
 (segment (start 114.17 99.98) (end 112.69 101.46) (width 0.2) (layer "B.Cu") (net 6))
 (segment (start 114.17 56.75) (end 114.17 99.98) (width 0.2) (layer "B.Cu") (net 6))
 (segment (start 108.38 53.3885) (end 107.545 53.3885) (width 0.2) (layer "F.Cu") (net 7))
 (segment (start 131.69 101.46) (end 132.060101 101.089899) (width 0.2) (layer "B.Cu") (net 7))
 (segment (start 116.027157 101.089899) (end 114.257056 102.86) (width 0.2) (layer "B.Cu") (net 7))
 (segment (start 132.060101 101.089899) (end 116.027157 101.089899) (width 0.2) (layer "B.Cu") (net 7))
 (segment (start 111.977056 102.86) (end 108.38 99.262944) (width 0.2) (layer "B.Cu") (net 7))
 (segment (start 114.257056 102.86) (end 111.977056 102.86) (width 0.2) (layer "B.Cu") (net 7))
 (segment (start 108.38 99.262944) (end 108.38 53.24) (width 0.2) (layer "B.Cu") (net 7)))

